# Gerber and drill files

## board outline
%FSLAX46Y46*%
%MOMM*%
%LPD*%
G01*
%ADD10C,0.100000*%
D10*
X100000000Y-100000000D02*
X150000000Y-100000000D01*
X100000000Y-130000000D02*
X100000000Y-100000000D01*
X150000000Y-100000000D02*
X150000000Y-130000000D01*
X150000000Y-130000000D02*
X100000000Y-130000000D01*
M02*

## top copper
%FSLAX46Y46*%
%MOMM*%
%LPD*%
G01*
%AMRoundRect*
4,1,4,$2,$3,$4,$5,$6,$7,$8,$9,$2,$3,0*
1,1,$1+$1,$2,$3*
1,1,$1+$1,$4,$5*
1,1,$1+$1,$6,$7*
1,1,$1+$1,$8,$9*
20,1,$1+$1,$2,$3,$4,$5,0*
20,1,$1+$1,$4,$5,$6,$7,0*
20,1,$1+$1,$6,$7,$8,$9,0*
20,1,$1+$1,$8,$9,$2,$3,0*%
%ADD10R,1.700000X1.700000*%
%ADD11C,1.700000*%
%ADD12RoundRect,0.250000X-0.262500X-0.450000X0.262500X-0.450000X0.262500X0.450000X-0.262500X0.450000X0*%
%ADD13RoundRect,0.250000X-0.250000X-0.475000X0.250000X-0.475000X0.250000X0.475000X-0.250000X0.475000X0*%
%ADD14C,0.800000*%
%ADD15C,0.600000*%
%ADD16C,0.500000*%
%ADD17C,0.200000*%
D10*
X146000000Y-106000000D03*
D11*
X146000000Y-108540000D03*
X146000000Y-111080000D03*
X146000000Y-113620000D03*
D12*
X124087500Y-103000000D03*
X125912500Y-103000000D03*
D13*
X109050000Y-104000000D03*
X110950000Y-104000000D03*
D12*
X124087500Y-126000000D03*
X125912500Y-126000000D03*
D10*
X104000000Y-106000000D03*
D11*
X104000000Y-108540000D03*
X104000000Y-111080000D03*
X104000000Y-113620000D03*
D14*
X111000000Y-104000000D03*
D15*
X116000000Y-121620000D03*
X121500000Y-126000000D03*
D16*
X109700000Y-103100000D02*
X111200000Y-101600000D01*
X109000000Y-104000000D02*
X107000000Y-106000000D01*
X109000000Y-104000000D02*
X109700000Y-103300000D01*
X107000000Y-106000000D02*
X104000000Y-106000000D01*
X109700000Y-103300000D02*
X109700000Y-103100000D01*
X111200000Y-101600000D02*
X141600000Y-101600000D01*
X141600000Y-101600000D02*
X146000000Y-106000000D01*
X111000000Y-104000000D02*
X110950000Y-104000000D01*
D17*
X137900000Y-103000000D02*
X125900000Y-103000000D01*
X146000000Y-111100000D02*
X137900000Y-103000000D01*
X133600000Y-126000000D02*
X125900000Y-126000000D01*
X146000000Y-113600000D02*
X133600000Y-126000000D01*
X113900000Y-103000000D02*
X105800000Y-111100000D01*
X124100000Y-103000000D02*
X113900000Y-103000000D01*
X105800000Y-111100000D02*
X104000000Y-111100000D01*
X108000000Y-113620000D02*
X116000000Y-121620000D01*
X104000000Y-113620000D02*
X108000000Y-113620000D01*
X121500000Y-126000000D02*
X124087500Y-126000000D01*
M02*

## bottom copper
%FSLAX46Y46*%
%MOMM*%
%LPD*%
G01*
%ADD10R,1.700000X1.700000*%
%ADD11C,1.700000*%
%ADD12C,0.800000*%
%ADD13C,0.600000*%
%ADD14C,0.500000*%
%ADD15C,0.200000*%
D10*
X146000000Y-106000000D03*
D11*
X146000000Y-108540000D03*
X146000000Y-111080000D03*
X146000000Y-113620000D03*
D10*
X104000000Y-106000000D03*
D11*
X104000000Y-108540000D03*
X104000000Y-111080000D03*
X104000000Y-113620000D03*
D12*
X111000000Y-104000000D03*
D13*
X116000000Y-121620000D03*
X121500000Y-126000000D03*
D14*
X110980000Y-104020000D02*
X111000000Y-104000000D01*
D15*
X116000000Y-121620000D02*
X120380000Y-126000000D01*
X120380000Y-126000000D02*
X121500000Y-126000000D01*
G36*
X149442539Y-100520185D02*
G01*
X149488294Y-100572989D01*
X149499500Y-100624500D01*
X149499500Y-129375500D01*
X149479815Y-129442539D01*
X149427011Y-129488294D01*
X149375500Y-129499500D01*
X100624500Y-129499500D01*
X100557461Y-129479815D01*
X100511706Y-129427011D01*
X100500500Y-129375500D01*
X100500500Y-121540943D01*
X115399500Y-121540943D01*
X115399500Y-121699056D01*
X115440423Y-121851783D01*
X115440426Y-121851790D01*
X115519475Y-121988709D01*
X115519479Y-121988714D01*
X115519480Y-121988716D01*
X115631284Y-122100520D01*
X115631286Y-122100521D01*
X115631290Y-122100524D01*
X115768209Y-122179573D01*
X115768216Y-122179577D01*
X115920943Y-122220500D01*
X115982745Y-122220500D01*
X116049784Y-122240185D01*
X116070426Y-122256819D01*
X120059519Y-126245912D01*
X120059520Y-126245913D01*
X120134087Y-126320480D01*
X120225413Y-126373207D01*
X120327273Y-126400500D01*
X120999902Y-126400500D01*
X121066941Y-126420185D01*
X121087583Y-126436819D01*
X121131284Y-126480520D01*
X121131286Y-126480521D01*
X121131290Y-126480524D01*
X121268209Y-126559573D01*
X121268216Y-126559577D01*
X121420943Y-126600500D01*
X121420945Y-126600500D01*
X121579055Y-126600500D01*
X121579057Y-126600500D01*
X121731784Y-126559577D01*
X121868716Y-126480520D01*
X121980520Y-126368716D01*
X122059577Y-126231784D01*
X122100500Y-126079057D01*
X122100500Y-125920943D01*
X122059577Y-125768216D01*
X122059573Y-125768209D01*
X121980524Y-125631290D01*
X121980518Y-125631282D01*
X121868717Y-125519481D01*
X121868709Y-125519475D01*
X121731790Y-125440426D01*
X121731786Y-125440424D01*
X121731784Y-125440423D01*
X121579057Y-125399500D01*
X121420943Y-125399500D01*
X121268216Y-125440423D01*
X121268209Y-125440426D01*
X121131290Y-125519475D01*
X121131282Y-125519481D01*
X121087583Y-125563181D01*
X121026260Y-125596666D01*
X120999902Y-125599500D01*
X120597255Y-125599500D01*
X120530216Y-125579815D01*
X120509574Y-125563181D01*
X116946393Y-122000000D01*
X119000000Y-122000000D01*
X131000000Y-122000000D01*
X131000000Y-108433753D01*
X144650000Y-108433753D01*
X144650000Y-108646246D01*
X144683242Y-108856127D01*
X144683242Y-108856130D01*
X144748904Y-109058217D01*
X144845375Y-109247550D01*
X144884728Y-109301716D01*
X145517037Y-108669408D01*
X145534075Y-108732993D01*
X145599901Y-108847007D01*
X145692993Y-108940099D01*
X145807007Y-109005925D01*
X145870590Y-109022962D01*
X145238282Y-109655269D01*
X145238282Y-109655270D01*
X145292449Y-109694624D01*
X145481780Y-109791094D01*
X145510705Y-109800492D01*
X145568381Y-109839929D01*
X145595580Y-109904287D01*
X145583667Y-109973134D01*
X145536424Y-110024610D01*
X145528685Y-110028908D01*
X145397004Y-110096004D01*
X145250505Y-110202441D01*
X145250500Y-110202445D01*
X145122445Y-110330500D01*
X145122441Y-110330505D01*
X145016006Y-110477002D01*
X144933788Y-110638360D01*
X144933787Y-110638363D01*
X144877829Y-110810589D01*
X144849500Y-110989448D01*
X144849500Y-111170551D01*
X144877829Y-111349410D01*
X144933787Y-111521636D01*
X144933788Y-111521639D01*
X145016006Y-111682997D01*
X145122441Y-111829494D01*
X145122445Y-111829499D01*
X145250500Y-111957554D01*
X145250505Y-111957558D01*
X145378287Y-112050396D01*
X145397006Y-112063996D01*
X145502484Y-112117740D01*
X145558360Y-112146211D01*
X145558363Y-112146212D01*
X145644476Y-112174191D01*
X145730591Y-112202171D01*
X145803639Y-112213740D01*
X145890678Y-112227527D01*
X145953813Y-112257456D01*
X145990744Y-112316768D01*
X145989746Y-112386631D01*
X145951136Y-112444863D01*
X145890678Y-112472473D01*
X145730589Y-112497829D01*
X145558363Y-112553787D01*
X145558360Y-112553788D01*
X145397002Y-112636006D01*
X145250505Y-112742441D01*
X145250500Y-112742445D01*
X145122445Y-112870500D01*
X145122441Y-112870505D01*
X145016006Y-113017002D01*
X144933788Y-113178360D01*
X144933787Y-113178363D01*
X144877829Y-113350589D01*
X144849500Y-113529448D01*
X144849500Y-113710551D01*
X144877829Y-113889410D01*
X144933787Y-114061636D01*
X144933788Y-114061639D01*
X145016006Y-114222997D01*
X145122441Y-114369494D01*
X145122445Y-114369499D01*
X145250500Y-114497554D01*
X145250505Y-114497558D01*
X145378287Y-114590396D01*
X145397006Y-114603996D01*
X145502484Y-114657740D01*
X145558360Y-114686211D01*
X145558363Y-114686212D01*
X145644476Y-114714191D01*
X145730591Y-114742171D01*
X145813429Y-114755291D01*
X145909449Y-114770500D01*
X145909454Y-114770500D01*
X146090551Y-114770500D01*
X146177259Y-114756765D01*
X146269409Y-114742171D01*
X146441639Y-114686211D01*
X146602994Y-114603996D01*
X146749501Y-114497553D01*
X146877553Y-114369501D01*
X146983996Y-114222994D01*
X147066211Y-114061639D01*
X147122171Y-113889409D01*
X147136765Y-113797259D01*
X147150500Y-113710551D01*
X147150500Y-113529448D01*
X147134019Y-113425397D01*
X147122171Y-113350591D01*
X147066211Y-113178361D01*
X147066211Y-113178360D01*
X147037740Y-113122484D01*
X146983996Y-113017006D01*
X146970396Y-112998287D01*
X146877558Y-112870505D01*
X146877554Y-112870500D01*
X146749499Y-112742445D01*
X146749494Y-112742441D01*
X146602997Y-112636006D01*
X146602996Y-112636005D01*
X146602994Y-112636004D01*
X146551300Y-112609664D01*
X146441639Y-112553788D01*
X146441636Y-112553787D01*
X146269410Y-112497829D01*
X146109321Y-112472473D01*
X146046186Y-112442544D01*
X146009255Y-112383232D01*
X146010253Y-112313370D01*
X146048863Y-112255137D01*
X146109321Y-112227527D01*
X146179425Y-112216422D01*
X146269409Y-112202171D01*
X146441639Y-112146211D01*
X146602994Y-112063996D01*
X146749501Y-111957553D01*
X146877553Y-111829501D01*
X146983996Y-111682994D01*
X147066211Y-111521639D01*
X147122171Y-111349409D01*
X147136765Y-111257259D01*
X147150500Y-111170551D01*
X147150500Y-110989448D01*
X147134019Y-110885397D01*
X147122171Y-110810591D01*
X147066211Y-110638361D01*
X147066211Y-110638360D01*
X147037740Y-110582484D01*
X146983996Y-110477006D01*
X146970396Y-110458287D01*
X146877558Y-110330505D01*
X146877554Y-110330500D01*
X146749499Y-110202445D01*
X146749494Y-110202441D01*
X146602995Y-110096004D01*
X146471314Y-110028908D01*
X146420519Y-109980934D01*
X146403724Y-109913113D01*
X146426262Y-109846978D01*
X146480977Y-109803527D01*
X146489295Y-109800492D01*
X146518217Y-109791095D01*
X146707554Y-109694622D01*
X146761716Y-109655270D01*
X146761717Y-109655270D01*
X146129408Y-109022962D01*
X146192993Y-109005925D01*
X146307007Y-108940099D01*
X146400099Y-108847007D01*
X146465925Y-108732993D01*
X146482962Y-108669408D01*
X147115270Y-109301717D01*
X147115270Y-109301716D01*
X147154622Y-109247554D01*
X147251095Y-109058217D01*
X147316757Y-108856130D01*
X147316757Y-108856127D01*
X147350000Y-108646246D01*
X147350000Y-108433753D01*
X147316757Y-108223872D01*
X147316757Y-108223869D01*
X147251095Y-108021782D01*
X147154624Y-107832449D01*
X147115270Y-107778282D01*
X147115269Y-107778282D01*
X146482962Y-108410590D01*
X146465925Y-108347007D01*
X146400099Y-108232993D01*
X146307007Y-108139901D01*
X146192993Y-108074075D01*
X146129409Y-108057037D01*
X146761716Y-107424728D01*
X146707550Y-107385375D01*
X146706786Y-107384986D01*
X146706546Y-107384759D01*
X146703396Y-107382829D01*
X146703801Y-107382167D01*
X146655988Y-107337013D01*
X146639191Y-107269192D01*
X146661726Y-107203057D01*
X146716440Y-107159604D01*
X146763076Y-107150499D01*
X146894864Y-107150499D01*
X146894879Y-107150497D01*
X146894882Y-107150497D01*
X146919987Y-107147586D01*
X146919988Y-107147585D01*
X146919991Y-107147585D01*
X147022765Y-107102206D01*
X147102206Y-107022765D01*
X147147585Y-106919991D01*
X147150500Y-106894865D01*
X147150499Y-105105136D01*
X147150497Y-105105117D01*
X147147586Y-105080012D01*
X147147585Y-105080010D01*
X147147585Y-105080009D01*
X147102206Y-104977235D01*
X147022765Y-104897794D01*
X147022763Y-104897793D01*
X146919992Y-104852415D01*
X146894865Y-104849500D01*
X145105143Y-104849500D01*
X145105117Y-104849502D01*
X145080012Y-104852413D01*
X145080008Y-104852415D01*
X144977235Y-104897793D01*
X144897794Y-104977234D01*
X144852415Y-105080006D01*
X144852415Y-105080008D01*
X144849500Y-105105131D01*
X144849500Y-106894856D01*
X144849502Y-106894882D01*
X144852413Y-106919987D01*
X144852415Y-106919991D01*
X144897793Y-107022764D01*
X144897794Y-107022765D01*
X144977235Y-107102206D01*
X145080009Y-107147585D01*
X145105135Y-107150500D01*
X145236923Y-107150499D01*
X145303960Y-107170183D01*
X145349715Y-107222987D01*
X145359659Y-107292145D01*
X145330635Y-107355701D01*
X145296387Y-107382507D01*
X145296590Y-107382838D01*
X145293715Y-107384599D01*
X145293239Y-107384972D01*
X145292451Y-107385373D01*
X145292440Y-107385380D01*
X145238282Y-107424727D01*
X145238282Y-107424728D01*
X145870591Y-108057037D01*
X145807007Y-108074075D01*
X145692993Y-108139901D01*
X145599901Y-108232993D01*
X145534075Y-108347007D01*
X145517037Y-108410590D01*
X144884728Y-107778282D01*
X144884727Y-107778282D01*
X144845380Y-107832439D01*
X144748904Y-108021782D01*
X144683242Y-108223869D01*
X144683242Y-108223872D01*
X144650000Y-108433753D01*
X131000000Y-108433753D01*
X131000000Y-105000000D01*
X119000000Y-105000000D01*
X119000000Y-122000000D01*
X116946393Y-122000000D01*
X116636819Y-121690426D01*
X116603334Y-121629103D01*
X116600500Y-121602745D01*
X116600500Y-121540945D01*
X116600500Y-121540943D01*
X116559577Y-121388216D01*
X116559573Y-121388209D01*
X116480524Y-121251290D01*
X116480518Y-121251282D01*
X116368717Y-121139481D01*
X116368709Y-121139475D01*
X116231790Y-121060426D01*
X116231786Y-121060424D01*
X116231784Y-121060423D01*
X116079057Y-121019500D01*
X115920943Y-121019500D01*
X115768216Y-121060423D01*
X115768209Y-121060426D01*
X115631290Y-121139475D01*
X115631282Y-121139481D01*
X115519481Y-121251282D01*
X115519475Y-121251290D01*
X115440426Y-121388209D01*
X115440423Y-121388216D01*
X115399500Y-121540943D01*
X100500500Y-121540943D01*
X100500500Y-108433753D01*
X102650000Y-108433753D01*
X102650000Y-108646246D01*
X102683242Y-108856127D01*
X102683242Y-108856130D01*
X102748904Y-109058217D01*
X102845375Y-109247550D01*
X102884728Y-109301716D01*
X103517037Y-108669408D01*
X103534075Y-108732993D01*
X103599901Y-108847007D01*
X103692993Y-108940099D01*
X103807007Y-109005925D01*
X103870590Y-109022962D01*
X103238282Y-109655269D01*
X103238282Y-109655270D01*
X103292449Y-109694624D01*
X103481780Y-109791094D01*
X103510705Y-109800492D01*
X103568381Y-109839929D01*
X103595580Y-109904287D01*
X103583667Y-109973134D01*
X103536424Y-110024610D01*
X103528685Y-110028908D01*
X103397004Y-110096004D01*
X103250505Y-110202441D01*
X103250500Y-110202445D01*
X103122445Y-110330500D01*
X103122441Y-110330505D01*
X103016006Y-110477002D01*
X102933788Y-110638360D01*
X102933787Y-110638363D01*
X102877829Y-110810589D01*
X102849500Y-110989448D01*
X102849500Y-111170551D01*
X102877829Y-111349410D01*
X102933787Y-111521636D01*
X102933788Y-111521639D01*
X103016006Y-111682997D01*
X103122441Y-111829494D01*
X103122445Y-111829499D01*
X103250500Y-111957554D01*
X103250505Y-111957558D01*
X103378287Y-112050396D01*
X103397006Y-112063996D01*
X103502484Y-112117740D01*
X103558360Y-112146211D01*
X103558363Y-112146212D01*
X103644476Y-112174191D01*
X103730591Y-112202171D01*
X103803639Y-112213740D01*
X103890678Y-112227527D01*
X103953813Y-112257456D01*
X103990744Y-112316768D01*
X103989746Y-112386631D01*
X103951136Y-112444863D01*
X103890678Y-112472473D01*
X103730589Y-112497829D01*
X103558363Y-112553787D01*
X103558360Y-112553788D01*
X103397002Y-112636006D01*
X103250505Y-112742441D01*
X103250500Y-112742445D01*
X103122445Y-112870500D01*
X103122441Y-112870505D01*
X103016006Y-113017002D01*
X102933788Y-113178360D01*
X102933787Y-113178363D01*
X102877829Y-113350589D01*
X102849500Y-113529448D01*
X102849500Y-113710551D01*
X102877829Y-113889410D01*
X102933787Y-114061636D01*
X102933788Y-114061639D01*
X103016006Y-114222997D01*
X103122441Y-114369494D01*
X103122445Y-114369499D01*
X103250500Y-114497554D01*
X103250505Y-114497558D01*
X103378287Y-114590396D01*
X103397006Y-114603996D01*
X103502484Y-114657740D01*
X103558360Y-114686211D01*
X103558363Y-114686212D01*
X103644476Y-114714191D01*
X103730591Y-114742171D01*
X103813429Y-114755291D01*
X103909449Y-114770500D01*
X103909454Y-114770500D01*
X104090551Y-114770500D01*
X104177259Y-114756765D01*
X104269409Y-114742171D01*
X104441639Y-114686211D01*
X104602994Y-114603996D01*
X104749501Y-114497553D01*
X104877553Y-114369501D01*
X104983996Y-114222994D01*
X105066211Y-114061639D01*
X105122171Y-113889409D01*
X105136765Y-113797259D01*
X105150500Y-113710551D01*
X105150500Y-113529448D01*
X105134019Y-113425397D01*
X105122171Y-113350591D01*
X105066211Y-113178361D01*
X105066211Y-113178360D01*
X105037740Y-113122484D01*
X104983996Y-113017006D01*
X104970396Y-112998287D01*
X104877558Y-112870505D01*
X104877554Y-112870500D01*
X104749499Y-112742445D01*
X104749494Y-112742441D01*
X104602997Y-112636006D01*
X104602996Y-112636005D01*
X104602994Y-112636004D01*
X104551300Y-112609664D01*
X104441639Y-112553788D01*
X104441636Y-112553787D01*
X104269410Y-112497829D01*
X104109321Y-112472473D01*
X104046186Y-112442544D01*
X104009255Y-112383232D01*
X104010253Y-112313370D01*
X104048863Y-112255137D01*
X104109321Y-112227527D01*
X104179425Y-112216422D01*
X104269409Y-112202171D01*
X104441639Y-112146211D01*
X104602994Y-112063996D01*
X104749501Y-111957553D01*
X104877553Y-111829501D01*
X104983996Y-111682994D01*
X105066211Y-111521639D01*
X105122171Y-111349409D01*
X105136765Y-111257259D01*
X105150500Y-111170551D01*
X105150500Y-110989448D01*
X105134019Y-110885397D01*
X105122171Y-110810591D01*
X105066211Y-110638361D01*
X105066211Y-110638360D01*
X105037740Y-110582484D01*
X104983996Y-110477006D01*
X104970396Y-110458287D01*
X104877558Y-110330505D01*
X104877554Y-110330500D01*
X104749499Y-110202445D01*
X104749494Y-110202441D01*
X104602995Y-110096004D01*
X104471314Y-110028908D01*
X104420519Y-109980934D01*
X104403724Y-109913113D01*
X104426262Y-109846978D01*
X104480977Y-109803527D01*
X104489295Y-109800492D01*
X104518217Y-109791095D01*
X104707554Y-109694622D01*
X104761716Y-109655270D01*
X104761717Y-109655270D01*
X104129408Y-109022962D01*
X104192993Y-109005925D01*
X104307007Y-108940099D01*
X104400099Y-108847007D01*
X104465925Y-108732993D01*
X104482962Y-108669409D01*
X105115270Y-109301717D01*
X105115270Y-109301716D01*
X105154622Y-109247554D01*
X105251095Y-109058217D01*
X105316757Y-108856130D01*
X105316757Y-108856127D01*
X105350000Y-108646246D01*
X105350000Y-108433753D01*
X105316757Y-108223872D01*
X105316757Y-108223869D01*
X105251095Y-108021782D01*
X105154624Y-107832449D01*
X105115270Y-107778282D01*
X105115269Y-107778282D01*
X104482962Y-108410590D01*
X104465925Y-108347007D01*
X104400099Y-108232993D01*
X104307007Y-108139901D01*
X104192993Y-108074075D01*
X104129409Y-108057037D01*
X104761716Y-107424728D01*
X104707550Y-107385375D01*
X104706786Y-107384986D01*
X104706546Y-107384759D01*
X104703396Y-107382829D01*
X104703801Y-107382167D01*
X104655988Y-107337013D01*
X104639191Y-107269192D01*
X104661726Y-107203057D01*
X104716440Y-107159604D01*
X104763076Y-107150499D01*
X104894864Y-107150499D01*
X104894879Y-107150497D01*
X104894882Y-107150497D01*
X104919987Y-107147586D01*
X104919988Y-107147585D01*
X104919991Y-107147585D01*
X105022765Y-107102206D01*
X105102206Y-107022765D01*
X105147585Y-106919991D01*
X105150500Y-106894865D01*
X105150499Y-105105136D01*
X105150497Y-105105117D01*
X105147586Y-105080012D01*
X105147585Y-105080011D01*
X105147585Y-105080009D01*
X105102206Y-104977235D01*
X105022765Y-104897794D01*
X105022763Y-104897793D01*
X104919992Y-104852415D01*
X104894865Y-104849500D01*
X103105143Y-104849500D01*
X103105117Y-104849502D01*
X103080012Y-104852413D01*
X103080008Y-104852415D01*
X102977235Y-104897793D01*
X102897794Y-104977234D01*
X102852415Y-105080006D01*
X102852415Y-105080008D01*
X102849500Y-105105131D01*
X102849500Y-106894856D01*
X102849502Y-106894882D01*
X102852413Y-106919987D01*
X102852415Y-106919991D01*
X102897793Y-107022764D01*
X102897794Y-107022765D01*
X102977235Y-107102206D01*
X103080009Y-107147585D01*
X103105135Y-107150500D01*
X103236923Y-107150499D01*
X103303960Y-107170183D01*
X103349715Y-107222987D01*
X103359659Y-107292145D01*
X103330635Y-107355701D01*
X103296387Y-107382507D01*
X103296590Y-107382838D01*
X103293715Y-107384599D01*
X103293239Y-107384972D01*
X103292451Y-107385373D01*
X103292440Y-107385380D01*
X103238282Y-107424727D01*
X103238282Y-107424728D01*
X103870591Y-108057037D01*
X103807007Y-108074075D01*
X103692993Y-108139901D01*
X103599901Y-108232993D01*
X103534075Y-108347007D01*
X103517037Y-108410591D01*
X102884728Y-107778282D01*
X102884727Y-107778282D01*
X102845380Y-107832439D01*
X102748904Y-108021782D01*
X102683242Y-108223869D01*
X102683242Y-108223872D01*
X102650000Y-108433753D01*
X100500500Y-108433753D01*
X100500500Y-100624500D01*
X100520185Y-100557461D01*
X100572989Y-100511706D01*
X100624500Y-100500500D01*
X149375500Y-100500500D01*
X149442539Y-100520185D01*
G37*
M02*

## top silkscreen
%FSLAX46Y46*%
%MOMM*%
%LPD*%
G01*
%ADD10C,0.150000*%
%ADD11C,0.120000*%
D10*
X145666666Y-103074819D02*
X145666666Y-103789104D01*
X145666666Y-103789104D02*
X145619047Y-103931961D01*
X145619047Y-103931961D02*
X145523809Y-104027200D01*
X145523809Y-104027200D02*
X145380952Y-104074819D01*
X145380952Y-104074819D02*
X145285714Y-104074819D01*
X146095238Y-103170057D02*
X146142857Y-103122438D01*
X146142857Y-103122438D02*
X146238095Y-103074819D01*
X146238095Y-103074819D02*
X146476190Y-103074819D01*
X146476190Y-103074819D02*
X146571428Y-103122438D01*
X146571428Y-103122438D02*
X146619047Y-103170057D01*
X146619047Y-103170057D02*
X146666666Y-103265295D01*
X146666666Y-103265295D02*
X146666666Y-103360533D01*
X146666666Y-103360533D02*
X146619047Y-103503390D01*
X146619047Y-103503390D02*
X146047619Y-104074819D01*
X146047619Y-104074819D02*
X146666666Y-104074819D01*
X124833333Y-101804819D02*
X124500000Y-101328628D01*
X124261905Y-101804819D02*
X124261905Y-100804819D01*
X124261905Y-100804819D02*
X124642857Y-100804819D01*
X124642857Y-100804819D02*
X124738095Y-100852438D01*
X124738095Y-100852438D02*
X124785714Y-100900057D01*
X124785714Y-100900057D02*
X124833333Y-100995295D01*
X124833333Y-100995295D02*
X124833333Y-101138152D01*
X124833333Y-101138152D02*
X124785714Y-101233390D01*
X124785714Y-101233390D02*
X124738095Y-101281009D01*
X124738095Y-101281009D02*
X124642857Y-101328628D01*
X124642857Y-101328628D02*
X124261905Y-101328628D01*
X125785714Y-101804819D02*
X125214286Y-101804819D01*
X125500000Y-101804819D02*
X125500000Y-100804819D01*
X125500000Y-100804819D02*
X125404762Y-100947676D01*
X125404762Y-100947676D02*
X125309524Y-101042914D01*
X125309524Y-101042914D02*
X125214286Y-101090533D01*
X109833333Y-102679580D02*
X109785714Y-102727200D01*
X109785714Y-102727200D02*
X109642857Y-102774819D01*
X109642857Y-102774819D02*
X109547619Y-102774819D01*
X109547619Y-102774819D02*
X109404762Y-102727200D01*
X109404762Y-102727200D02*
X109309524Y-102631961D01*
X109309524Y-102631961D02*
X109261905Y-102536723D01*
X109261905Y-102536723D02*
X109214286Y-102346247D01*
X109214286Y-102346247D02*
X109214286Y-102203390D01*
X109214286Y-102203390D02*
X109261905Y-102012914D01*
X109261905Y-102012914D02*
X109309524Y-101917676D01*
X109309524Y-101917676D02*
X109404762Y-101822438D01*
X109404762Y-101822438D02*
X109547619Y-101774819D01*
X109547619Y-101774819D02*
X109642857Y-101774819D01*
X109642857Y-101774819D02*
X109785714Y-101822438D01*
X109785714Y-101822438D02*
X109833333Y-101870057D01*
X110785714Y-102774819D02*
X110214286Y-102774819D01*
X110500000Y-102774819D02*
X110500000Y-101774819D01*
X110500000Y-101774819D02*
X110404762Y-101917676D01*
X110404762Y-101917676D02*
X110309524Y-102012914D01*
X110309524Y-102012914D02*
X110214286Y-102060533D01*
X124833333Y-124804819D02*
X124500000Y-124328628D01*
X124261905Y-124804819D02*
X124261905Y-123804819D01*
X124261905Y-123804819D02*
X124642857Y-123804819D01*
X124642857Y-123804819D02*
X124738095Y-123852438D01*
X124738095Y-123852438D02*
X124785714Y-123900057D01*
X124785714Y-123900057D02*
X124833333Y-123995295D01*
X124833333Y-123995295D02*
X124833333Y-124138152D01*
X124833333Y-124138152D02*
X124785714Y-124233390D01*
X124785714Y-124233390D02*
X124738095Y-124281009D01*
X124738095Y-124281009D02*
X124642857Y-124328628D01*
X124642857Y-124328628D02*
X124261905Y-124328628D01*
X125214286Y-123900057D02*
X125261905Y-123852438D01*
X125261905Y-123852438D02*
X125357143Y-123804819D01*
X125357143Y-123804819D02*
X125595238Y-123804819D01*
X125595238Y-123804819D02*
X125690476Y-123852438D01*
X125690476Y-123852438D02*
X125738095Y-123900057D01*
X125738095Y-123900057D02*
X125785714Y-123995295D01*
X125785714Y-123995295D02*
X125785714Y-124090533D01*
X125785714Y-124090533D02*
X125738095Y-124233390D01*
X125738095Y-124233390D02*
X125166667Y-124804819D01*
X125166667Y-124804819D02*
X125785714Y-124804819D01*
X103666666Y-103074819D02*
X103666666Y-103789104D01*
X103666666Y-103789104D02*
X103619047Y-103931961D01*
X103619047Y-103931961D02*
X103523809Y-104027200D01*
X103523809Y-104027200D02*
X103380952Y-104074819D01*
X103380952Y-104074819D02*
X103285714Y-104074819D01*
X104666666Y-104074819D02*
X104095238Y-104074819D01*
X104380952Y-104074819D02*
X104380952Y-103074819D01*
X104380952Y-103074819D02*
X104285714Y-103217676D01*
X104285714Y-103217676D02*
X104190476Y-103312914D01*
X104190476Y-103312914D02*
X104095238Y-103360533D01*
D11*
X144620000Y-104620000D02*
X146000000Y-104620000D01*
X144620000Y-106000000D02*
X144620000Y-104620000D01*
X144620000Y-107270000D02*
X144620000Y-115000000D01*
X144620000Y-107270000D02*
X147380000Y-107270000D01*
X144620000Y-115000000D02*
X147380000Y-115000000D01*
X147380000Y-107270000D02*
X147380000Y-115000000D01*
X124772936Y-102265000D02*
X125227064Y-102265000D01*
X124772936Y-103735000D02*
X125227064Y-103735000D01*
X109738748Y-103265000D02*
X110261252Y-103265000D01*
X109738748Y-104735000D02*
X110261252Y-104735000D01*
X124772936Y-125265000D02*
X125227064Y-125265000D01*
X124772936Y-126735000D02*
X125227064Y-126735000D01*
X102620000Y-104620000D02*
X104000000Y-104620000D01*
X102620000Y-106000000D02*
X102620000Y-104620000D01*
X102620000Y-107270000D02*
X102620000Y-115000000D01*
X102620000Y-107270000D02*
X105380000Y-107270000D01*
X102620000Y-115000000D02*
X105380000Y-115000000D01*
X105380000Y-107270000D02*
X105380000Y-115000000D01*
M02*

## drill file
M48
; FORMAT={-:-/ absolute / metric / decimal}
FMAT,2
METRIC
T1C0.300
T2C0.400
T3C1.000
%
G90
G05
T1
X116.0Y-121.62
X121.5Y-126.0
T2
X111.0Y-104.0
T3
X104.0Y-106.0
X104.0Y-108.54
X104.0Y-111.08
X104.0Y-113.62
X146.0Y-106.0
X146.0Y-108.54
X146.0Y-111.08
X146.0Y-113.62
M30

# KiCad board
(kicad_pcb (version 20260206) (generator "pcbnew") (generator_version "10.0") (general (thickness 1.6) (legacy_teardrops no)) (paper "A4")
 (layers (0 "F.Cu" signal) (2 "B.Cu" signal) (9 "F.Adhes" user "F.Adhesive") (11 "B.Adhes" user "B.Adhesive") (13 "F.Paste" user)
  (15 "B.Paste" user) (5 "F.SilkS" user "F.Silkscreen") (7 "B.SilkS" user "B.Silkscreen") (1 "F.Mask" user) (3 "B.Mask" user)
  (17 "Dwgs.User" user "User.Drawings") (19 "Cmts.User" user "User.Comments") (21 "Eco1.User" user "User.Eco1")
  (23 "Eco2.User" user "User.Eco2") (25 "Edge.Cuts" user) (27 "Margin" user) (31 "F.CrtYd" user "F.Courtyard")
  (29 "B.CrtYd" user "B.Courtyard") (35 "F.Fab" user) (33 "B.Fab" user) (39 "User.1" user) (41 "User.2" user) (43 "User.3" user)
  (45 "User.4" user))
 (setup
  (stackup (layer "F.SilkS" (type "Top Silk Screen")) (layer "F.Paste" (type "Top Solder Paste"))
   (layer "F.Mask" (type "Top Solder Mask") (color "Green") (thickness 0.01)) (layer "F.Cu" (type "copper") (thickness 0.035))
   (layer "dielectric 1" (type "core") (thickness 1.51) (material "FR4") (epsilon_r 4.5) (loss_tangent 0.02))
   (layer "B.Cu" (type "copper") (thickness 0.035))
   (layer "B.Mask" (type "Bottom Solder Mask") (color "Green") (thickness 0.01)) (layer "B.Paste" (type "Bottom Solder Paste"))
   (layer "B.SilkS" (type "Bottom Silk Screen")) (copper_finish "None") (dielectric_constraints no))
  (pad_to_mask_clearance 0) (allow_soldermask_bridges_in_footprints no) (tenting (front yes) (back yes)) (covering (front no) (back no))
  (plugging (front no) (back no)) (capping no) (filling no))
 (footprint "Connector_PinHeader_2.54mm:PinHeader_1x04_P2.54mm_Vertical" (layer "F.Cu") (at 146 106)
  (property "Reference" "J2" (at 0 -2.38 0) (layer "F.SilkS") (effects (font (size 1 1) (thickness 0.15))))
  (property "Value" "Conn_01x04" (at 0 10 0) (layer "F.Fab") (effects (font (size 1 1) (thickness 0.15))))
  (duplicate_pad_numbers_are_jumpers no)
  (fp_line (start -1.38 -1.38) (end 0 -1.38) (stroke (width 0.12) (type solid)) (layer "F.SilkS"))
  (fp_line (start -1.38 0) (end -1.38 -1.38) (stroke (width 0.12) (type solid)) (layer "F.SilkS"))
  (fp_line (start -1.38 1.27) (end -1.38 9) (stroke (width 0.12) (type solid)) (layer "F.SilkS"))
  (fp_line (start -1.38 1.27) (end 1.38 1.27) (stroke (width 0.12) (type solid)) (layer "F.SilkS"))
  (fp_line (start -1.38 9) (end 1.38 9) (stroke (width 0.12) (type solid)) (layer "F.SilkS"))
  (fp_line (start 1.38 1.27) (end 1.38 9) (stroke (width 0.12) (type solid)) (layer "F.SilkS"))
  (pad "1" thru_hole rect (at 0 0) (size 1.7 1.7) (drill 1) (layers "*.Cu" "*.Mask") (remove_unused_layers no) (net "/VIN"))
  (pad "2" thru_hole circle (at 0 2.54) (size 1.7 1.7) (drill 1) (layers "*.Cu" "*.Mask") (remove_unused_layers no) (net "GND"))
  (pad "3" thru_hole circle (at 0 5.08) (size 1.7 1.7) (drill 1) (layers "*.Cu" "*.Mask") (remove_unused_layers no) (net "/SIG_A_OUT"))
  (pad "4" thru_hole circle (at 0 7.62) (size 1.7 1.7) (drill 1) (layers "*.Cu" "*.Mask") (remove_unused_layers no) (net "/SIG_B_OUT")))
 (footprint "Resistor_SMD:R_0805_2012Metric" (layer "F.Cu") (at 125 103)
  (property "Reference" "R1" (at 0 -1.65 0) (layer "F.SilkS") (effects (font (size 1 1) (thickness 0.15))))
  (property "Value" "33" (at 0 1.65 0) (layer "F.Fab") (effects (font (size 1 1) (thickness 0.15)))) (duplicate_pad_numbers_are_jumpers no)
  (fp_line (start -0.227064 -0.735) (end 0.227064 -0.735) (stroke (width 0.12) (type solid)) (layer "F.SilkS"))
  (fp_line (start -0.227064 0.735) (end 0.227064 0.735) (stroke (width 0.12) (type solid)) (layer "F.SilkS"))
  (pad "1" smd roundrect (at -0.9125 0) (size 1.025 1.4) (layers "F.Cu" "F.Mask" "F.Paste") (roundrect_rratio 0.243902) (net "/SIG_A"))
  (pad "2" smd roundrect (at 0.9125 0) (size 1.025 1.4) (layers "F.Cu" "F.Mask" "F.Paste") (roundrect_rratio 0.243902) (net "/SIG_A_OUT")))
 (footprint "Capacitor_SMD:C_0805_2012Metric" (layer "F.Cu") (at 110 104)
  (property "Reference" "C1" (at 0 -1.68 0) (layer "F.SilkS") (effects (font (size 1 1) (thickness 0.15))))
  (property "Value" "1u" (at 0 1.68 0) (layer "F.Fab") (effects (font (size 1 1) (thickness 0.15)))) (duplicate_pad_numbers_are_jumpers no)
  (fp_line (start -0.261252 -0.735) (end 0.261252 -0.735) (stroke (width 0.12) (type solid)) (layer "F.SilkS"))
  (fp_line (start -0.261252 0.735) (end 0.261252 0.735) (stroke (width 0.12) (type solid)) (layer "F.SilkS"))
  (pad "1" smd roundrect (at -0.95 0) (size 1 1.45) (layers "F.Cu" "F.Mask" "F.Paste") (roundrect_rratio 0.25) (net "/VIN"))
  (pad "2" smd roundrect (at 0.95 0) (size 1 1.45) (layers "F.Cu" "F.Mask" "F.Paste") (roundrect_rratio 0.25) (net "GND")))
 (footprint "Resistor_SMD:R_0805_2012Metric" (layer "F.Cu") (at 125 126)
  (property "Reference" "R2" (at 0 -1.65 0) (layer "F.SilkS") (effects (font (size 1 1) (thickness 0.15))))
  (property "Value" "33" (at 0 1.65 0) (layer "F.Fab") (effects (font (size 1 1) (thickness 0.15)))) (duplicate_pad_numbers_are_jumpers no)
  (fp_line (start -0.227064 -0.735) (end 0.227064 -0.735) (stroke (width 0.12) (type solid)) (layer "F.SilkS"))
  (fp_line (start -0.227064 0.735) (end 0.227064 0.735) (stroke (width 0.12) (type solid)) (layer "F.SilkS"))
  (pad "1" smd roundrect (at -0.9125 0) (size 1.025 1.4) (layers "F.Cu" "F.Mask" "F.Paste") (roundrect_rratio 0.243902) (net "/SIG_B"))
  (pad "2" smd roundrect (at 0.9125 0) (size 1.025 1.4) (layers "F.Cu" "F.Mask" "F.Paste") (roundrect_rratio 0.243902) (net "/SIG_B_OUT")))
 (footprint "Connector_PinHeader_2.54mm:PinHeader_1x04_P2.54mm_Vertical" (layer "F.Cu") (at 104 106)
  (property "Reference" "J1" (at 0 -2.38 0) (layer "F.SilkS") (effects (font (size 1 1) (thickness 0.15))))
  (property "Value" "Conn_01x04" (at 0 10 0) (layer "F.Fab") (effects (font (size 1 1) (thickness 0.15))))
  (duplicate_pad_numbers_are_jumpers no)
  (fp_line (start -1.38 -1.38) (end 0 -1.38) (stroke (width 0.12) (type solid)) (layer "F.SilkS"))
  (fp_line (start -1.38 0) (end -1.38 -1.38) (stroke (width 0.12) (type solid)) (layer "F.SilkS"))
  (fp_line (start -1.38 1.27) (end -1.38 9) (stroke (width 0.12) (type solid)) (layer "F.SilkS"))
  (fp_line (start -1.38 1.27) (end 1.38 1.27) (stroke (width 0.12) (type solid)) (layer "F.SilkS"))
  (fp_line (start -1.38 9) (end 1.38 9) (stroke (width 0.12) (type solid)) (layer "F.SilkS"))
  (fp_line (start 1.38 1.27) (end 1.38 9) (stroke (width 0.12) (type solid)) (layer "F.SilkS"))
  (pad "1" thru_hole rect (at 0 0) (size 1.7 1.7) (drill 1) (layers "*.Cu" "*.Mask") (remove_unused_layers no) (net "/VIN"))
  (pad "2" thru_hole circle (at 0 2.54) (size 1.7 1.7) (drill 1) (layers "*.Cu" "*.Mask") (remove_unused_layers no) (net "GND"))
  (pad "3" thru_hole circle (at 0 5.08) (size 1.7 1.7) (drill 1) (layers "*.Cu" "*.Mask") (remove_unused_layers no) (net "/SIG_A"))
  (pad "4" thru_hole circle (at 0 7.62) (size 1.7 1.7) (drill 1) (layers "*.Cu" "*.Mask") (remove_unused_layers no) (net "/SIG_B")))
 (gr_line (start 100 100) (end 150 100) (stroke (width 0.1) (type default)) (layer "Edge.Cuts"))
 (gr_line (start 100 130) (end 100 100) (stroke (width 0.1) (type default)) (layer "Edge.Cuts"))
 (gr_line (start 150 100) (end 150 130) (stroke (width 0.1) (type default)) (layer "Edge.Cuts"))
 (gr_line (start 150 130) (end 100 130) (stroke (width 0.1) (type default)) (layer "Edge.Cuts"))
 (segment (start 109.7 103.1) (end 111.2 101.6) (width 0.5) (layer "F.Cu") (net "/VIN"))
 (segment (start 109 104) (end 107 106) (width 0.5) (layer "F.Cu") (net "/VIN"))
 (segment (start 109 104) (end 109.7 103.3) (width 0.5) (layer "F.Cu") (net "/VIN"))
 (segment (start 107 106) (end 104 106) (width 0.5) (layer "F.Cu") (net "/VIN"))
 (segment (start 109.7 103.3) (end 109.7 103.1) (width 0.5) (layer "F.Cu") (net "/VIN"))
 (segment (start 111.2 101.6) (end 141.6 101.6) (width 0.5) (layer "F.Cu") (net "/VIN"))
 (segment (start 141.6 101.6) (end 146 106) (width 0.5) (layer "F.Cu") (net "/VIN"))
 (segment (start 111 104) (end 110.95 104) (width 0.5) (layer "F.Cu") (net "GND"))
 (via (at 111 104) (size 0.8) (drill 0.4) (layers "F.Cu" "B.Cu") (capping yes) (filling yes) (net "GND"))
 (segment (start 110.98 104.02) (end 111 104) (width 0.5) (layer "B.Cu") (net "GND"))
 (segment (start 137.9 103) (end 125.9 103) (width 0.2) (layer "F.Cu") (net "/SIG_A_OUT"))
 (segment (start 146 111.1) (end 137.9 103) (width 0.2) (layer "F.Cu") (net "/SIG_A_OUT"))
 (segment (start 133.6 126) (end 125.9 126) (width 0.2) (layer "F.Cu") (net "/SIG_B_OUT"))
 (segment (start 146 113.6) (end 133.6 126) (width 0.2) (layer "F.Cu") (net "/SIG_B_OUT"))
 (segment (start 113.9 103) (end 105.8 111.1) (width 0.2) (layer "F.Cu") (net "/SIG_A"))
 (segment (start 124.1 103) (end 113.9 103) (width 0.2) (layer "F.Cu") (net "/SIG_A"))
 (segment (start 105.8 111.1) (end 104 111.1) (width 0.2) (layer "F.Cu") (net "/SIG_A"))
 (segment (start 108 113.62) (end 116 121.62) (width 0.2) (locked yes) (layer "F.Cu") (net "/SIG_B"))
 (segment (start 104 113.62) (end 108 113.62) (width 0.2) (locked yes) (layer "F.Cu") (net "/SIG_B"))
 (segment (start 121.5 126) (end 124.0875 126) (width 0.2) (locked yes) (layer "F.Cu") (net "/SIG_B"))
 (via (at 116 121.62) (size 0.6) (drill 0.3) (layers "F.Cu" "B.Cu") (locked yes) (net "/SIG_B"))
 (via (at 121.5 126) (size 0.6) (drill 0.3) (layers "F.Cu" "B.Cu") (locked yes) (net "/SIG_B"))
 (segment (start 116 121.62) (end 120.38 126) (width 0.2) (locked yes) (layer "B.Cu") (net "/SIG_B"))
 (segment (start 120.38 126) (end 121.5 126) (width 0.2) (locked yes) (layer "B.Cu") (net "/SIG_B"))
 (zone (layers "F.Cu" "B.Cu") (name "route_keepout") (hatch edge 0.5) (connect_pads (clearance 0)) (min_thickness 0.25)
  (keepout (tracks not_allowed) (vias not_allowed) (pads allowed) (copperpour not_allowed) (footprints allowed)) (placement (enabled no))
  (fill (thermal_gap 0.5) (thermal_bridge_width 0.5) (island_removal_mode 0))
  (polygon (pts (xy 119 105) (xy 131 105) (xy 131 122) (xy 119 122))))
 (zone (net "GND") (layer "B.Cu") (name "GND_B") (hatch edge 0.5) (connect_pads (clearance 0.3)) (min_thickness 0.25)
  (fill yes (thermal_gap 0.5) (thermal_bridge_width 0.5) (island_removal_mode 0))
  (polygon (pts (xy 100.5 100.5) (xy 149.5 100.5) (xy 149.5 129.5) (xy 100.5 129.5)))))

